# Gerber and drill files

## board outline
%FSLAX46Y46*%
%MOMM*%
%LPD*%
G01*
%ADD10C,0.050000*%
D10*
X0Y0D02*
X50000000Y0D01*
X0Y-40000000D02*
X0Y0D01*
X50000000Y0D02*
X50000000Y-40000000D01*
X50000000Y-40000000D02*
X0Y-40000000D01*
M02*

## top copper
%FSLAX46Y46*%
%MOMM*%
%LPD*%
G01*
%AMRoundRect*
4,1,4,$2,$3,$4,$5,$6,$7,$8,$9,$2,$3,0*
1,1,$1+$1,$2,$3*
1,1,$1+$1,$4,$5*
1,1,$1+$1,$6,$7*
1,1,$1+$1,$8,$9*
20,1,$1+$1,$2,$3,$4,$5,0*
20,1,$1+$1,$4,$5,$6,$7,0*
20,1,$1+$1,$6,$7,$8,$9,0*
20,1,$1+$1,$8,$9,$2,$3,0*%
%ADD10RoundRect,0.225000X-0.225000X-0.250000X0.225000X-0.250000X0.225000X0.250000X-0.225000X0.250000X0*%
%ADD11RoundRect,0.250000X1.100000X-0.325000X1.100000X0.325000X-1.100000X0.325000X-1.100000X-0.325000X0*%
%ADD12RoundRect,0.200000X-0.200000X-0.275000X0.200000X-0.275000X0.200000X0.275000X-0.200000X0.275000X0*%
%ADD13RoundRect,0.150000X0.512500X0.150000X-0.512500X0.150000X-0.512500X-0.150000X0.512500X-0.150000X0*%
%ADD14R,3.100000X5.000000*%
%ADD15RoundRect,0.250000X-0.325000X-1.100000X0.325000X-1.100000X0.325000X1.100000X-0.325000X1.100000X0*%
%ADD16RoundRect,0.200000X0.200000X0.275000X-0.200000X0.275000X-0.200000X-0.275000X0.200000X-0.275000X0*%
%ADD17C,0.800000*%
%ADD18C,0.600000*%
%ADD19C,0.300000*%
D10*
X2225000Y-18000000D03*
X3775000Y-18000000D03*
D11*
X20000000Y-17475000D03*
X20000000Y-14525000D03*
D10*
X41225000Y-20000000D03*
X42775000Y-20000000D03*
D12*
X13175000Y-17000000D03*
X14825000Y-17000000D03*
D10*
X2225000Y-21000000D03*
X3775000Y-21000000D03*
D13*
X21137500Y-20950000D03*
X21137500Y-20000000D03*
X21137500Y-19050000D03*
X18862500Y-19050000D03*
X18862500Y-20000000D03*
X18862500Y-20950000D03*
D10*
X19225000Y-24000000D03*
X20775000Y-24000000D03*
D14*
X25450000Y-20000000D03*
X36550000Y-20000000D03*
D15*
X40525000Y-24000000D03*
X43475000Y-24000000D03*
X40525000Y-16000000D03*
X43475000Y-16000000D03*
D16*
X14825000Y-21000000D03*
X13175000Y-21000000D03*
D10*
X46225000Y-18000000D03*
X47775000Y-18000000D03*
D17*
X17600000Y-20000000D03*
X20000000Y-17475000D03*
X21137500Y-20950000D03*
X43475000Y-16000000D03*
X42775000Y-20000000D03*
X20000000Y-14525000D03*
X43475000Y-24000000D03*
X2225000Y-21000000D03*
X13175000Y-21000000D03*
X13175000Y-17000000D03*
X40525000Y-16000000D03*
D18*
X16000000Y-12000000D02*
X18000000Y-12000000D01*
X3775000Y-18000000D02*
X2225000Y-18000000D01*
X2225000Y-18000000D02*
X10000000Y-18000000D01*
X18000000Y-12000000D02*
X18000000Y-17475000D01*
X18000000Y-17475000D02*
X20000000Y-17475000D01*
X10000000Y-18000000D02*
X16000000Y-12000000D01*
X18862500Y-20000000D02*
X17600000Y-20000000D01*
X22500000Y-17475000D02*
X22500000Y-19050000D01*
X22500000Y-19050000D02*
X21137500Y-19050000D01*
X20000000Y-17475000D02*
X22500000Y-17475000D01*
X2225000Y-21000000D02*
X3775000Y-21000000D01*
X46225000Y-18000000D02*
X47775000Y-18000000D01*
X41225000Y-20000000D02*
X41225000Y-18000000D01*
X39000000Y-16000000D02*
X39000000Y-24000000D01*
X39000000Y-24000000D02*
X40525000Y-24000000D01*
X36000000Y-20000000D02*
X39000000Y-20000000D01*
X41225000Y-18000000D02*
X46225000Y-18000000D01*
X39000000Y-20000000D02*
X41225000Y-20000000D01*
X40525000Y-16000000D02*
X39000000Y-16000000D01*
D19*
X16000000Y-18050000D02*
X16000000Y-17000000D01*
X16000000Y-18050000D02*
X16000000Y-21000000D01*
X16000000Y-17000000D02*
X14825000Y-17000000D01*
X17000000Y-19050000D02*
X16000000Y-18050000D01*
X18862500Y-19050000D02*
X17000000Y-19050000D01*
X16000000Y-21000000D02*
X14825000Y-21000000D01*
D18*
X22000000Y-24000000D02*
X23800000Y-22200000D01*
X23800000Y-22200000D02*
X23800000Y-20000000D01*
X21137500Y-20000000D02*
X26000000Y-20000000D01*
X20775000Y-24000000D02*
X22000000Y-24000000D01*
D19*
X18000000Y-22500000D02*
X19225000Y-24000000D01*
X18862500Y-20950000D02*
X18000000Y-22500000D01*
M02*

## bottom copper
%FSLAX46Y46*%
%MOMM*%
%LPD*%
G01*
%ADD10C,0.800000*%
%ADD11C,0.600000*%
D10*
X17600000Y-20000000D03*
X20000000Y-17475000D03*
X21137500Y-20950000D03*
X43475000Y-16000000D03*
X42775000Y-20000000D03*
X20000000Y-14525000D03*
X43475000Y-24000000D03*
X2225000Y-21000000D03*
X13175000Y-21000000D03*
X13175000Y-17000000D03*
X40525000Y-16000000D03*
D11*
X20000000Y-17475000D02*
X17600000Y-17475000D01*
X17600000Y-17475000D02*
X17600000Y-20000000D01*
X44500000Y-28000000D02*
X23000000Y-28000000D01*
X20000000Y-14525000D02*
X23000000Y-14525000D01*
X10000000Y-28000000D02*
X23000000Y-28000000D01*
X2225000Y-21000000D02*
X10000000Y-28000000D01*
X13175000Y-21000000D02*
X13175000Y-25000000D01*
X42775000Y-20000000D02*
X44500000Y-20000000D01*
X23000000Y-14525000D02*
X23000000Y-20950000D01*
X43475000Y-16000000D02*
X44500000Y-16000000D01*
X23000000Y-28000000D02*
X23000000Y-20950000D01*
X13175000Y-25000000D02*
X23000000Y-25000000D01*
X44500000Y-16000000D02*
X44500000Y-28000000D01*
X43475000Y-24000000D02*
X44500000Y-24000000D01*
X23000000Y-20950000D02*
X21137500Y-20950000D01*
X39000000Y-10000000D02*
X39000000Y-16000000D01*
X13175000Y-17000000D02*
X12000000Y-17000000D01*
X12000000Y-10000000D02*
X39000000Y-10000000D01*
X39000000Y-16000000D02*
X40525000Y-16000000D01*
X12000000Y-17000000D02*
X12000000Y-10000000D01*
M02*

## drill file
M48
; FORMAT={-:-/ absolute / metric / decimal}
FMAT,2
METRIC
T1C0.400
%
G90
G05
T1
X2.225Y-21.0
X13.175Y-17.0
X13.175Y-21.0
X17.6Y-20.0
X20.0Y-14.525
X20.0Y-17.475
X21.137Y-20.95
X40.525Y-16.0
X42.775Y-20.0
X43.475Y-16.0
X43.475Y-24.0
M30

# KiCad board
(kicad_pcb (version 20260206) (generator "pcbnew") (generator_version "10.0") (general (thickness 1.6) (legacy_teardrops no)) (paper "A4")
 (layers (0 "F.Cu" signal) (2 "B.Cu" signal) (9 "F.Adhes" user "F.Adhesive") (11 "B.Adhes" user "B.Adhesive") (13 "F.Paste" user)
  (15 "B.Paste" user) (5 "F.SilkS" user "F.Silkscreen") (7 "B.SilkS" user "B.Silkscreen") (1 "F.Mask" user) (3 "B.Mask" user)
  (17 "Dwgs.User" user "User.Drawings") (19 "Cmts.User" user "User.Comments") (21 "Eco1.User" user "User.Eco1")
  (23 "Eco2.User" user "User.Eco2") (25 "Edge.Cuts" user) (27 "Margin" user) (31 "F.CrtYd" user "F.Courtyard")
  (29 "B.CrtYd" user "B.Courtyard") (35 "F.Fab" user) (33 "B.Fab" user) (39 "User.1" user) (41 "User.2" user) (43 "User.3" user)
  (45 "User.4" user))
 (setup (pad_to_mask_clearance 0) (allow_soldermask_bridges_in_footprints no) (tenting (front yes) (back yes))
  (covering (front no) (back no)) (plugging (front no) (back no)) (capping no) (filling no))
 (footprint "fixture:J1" (layer "F.Cu") (at 3 18)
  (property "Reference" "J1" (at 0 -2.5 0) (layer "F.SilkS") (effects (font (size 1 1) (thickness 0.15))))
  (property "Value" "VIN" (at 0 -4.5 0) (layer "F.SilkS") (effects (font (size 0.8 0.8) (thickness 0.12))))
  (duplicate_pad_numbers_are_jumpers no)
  (pad "1" smd roundrect (at -0.775 0) (size 0.9 0.95) (layers "F.Cu" "F.Mask" "F.Paste") (roundrect_rratio 0.25) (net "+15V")
   (thermal_bridge_angle 45))
  (pad "2" smd roundrect (at 0.775 0) (size 0.9 0.95) (layers "F.Cu" "F.Mask" "F.Paste") (roundrect_rratio 0.25) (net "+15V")
   (thermal_bridge_angle 45)))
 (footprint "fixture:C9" (layer "F.Cu") (at 20 16 90)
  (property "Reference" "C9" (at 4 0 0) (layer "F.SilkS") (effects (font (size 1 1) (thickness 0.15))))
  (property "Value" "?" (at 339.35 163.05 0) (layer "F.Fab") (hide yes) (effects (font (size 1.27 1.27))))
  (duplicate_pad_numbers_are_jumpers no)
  (pad "1" smd roundrect (at -1.475 0 90) (size 1.15 2.7) (layers "F.Cu" "F.Mask" "F.Paste") (roundrect_rratio 0.217391) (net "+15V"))
  (pad "2" smd roundrect (at 1.475 0 90) (size 1.15 2.7) (layers "F.Cu" "F.Mask" "F.Paste") (roundrect_rratio 0.217391) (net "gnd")))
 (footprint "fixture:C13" (layer "F.Cu") (at 42 20)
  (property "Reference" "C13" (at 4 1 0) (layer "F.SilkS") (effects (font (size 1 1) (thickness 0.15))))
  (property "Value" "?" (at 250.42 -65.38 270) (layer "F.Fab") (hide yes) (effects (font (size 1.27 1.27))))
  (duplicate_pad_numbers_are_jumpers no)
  (pad "1" smd roundrect (at -0.775 0) (size 0.9 0.95) (layers "F.Cu" "F.Mask" "F.Paste") (roundrect_rratio 0.25) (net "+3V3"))
  (pad "2" smd roundrect (at 0.775 0) (size 0.9 0.95) (layers "F.Cu" "F.Mask" "F.Paste") (roundrect_rratio 0.25) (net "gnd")))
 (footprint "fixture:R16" (layer "F.Cu") (at 14 17)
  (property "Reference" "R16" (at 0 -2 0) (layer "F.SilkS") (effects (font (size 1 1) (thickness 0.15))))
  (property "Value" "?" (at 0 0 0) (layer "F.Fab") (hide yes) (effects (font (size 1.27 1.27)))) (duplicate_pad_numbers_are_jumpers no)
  (pad "1" smd roundrect (at -0.825 0) (size 0.8 0.95) (layers "F.Cu" "F.Mask" "F.Paste") (roundrect_rratio 0.25) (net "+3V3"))
  (pad "2" smd roundrect (at 0.825 0) (size 0.8 0.95) (layers "F.Cu" "F.Mask" "F.Paste") (roundrect_rratio 0.25) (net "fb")))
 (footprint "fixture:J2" (layer "F.Cu") (at 3 21)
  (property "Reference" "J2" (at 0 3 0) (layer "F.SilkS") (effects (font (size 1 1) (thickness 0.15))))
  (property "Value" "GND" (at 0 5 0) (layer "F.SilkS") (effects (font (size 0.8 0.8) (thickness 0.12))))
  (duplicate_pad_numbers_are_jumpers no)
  (pad "1" smd roundrect (at -0.775 0) (size 0.9 0.95) (layers "F.Cu" "F.Mask" "F.Paste") (roundrect_rratio 0.25) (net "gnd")
   (thermal_bridge_angle 45))
  (pad "2" smd roundrect (at 0.775 0) (size 0.9 0.95) (layers "F.Cu" "F.Mask" "F.Paste") (roundrect_rratio 0.25) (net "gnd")
   (thermal_bridge_angle 45)))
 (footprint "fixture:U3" (layer "F.Cu") (at 20 20 180)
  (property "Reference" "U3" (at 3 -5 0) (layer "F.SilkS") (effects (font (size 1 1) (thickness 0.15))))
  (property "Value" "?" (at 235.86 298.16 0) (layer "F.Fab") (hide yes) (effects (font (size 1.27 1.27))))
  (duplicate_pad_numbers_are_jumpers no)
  (pad "1" smd roundrect (at -1.1375 -0.95 180) (size 1.325 0.6) (layers "F.Cu" "F.Mask" "F.Paste") (roundrect_rratio 0.25) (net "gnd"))
  (pad "2" smd roundrect (at -1.1375 0 180) (size 1.325 0.6) (layers "F.Cu" "F.Mask" "F.Paste") (roundrect_rratio 0.25) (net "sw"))
  (pad "3" smd roundrect (at -1.1375 0.95 180) (size 1.325 0.6) (layers "F.Cu" "F.Mask" "F.Paste") (roundrect_rratio 0.25) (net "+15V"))
  (pad "4" smd roundrect (at 1.1375 0.95 180) (size 1.325 0.6) (layers "F.Cu" "F.Mask" "F.Paste") (roundrect_rratio 0.25) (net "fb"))
  (pad "5" smd roundrect (at 1.1375 0 180) (size 1.325 0.6) (layers "F.Cu" "F.Mask" "F.Paste") (roundrect_rratio 0.25) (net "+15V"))
  (pad "6" smd roundrect (at 1.1375 -0.95 180) (size 1.325 0.6) (layers "F.Cu" "F.Mask" "F.Paste") (roundrect_rratio 0.25) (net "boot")))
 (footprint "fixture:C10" (layer "F.Cu") (at 20 24)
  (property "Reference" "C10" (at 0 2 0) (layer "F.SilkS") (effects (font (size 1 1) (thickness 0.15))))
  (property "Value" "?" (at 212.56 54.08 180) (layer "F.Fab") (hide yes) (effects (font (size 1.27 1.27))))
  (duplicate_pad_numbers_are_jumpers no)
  (pad "1" smd roundrect (at -0.775 0) (size 0.9 0.95) (layers "F.Cu" "F.Mask" "F.Paste") (roundrect_rratio 0.25) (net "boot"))
  (pad "2" smd roundrect (at 0.775 0) (size 0.9 0.95) (layers "F.Cu" "F.Mask" "F.Paste") (roundrect_rratio 0.25) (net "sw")))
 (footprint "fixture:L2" (layer "F.Cu") (at 31 20)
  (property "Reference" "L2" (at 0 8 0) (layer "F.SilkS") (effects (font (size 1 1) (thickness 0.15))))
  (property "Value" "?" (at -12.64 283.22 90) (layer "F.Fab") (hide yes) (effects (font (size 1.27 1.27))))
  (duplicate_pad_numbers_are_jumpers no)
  (pad "1" smd rect (at -5.55 0) (size 3.1 5.0) (layers "F.Cu" "F.Mask" "F.Paste") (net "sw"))
  (pad "2" smd rect (at 5.55 0) (size 3.1 5.0) (layers "F.Cu" "F.Mask" "F.Paste") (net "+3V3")))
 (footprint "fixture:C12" (layer "F.Cu") (at 42 24)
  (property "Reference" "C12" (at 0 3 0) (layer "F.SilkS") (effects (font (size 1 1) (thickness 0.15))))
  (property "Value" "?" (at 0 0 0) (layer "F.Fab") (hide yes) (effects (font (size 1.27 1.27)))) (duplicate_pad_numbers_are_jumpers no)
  (pad "1" smd roundrect (at -1.475 0) (size 1.15 2.7) (layers "F.Cu" "F.Mask" "F.Paste") (roundrect_rratio 0.217391) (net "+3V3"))
  (pad "2" smd roundrect (at 1.475 0) (size 1.15 2.7) (layers "F.Cu" "F.Mask" "F.Paste") (roundrect_rratio 0.217391) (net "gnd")))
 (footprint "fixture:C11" (layer "F.Cu") (at 42 16)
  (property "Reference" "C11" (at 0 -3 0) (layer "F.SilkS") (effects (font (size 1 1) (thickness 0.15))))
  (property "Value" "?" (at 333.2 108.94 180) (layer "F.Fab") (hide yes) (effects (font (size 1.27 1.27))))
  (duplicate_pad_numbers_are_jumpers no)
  (pad "1" smd roundrect (at -1.475 0) (size 1.15 2.7) (layers "F.Cu" "F.Mask" "F.Paste") (roundrect_rratio 0.217391) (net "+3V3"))
  (pad "2" smd roundrect (at 1.475 0) (size 1.15 2.7) (layers "F.Cu" "F.Mask" "F.Paste") (roundrect_rratio 0.217391) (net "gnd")))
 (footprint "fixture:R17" (layer "F.Cu") (at 14 21 180)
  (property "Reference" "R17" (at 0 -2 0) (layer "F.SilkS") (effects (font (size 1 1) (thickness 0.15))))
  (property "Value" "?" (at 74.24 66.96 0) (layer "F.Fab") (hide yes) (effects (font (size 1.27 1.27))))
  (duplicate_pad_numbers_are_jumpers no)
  (pad "1" smd roundrect (at -0.825 0 180) (size 0.8 0.95) (layers "F.Cu" "F.Mask" "F.Paste") (roundrect_rratio 0.25) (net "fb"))
  (pad "2" smd roundrect (at 0.825 0 180) (size 0.8 0.95) (layers "F.Cu" "F.Mask" "F.Paste") (roundrect_rratio 0.25) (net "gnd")))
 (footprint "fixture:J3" (layer "F.Cu") (at 47 18)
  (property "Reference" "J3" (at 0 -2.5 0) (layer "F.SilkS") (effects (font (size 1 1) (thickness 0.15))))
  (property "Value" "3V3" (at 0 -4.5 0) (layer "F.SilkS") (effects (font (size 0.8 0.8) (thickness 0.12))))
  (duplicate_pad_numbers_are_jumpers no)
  (pad "1" smd roundrect (at -0.775 0) (size 0.9 0.95) (layers "F.Cu" "F.Mask" "F.Paste") (roundrect_rratio 0.25) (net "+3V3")
   (thermal_bridge_angle 45))
  (pad "2" smd roundrect (at 0.775 0) (size 0.9 0.95) (layers "F.Cu" "F.Mask" "F.Paste") (roundrect_rratio 0.25) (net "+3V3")
   (thermal_bridge_angle 45)))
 (gr_line (start 0 0) (end 50 0) (stroke (width 0.05) (type default)) (layer "Edge.Cuts"))
 (gr_line (start 0 40) (end 0 0) (stroke (width 0.05) (type default)) (layer "Edge.Cuts"))
 (gr_line (start 50 0) (end 50 40) (stroke (width 0.05) (type default)) (layer "Edge.Cuts"))
 (gr_line (start 50 40) (end 0 40) (stroke (width 0.05) (type default)) (layer "Edge.Cuts"))
 (segment (start 16 12) (end 18 12) (width 0.6) (layer "F.Cu") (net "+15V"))
 (segment (start 3.775 18) (end 2.225 18) (width 0.6) (layer "F.Cu") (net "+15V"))
 (segment (start 2.225 18) (end 10 18) (width 0.6) (layer "F.Cu") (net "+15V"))
 (segment (start 18 12) (end 18 17.475) (width 0.6) (layer "F.Cu") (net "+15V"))
 (segment (start 18 17.475) (end 20 17.475) (width 0.6) (layer "F.Cu") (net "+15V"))
 (segment (start 10 18) (end 16 12) (width 0.6) (layer "F.Cu") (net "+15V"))
 (segment (start 18.8625 20) (end 17.6 20) (width 0.6) (layer "F.Cu") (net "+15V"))
 (segment (start 22.5 17.475) (end 22.5 19.05) (width 0.6) (layer "F.Cu") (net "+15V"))
 (segment (start 22.5 19.05) (end 21.1375 19.05) (width 0.6) (layer "F.Cu") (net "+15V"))
 (segment (start 20 17.475) (end 22.5 17.475) (width 0.6) (layer "F.Cu") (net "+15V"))
 (via (at 17.6 20) (size 0.8) (drill 0.4) (layers "F.Cu" "B.Cu") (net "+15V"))
 (via (at 20 17.475) (size 0.8) (drill 0.4) (layers "F.Cu" "B.Cu") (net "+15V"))
 (segment (start 20 17.475) (end 17.6 17.475) (width 0.6) (layer "B.Cu") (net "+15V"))
 (segment (start 17.6 17.475) (end 17.6 20) (width 0.6) (layer "B.Cu") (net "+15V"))
 (segment (start 2.225 21) (end 3.775 21) (width 0.6) (layer "F.Cu") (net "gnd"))
 (via (at 21.1375 20.95) (size 0.8) (drill 0.4) (layers "F.Cu" "B.Cu") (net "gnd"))
 (via (at 43.475 16) (size 0.8) (drill 0.4) (layers "F.Cu" "B.Cu") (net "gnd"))
 (via (at 42.775 20) (size 0.8) (drill 0.4) (layers "F.Cu" "B.Cu") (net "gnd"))
 (via (at 20 14.525) (size 0.8) (drill 0.4) (layers "F.Cu" "B.Cu") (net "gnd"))
 (via (at 43.475 24) (size 0.8) (drill 0.4) (layers "F.Cu" "B.Cu") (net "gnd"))
 (via (at 2.225 21) (size 0.8) (drill 0.4) (layers "F.Cu" "B.Cu") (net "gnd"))
 (via (at 13.175 21) (size 0.8) (drill 0.4) (layers "F.Cu" "B.Cu") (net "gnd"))
 (segment (start 44.5 28) (end 23 28) (width 0.6) (layer "B.Cu") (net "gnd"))
 (segment (start 20 14.525) (end 23 14.525) (width 0.6) (layer "B.Cu") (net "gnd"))
 (segment (start 10 28) (end 23 28) (width 0.6) (layer "B.Cu") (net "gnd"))
 (segment (start 2.225 21) (end 10 28) (width 0.6) (layer "B.Cu") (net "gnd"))
 (segment (start 13.175 21) (end 13.175 25) (width 0.6) (layer "B.Cu") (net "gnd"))
 (segment (start 42.775 20) (end 44.5 20) (width 0.6) (layer "B.Cu") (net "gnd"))
 (segment (start 23 14.525) (end 23 20.95) (width 0.6) (layer "B.Cu") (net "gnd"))
 (segment (start 43.475 16) (end 44.5 16) (width 0.6) (layer "B.Cu") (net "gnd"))
 (segment (start 23 28) (end 23 20.95) (width 0.6) (layer "B.Cu") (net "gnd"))
 (segment (start 13.175 25) (end 23 25) (width 0.6) (layer "B.Cu") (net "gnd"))
 (segment (start 44.5 16) (end 44.5 28) (width 0.6) (layer "B.Cu") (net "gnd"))
 (segment (start 43.475 24) (end 44.5 24) (width 0.6) (layer "B.Cu") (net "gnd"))
 (segment (start 23 20.95) (end 21.1375 20.95) (width 0.6) (layer "B.Cu") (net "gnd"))
 (segment (start 46.225 18) (end 47.775 18) (width 0.6) (layer "F.Cu") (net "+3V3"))
 (segment (start 41.225 20) (end 41.225 18) (width 0.6) (layer "F.Cu") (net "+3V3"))
 (segment (start 39 16) (end 39 24) (width 0.6) (layer "F.Cu") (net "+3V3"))
 (segment (start 39 24) (end 40.525 24) (width 0.6) (layer "F.Cu") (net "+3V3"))
 (segment (start 36 20) (end 39 20) (width 0.6) (layer "F.Cu") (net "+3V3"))
 (segment (start 41.225 18) (end 46.225 18) (width 0.6) (layer "F.Cu") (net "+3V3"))
 (segment (start 39 20) (end 41.225 20) (width 0.6) (layer "F.Cu") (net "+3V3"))
 (segment (start 40.525 16) (end 39 16) (width 0.6) (layer "F.Cu") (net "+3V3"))
 (via (at 13.175 17) (size 0.8) (drill 0.4) (layers "F.Cu" "B.Cu") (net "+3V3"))
 (via (at 40.525 16) (size 0.8) (drill 0.4) (layers "F.Cu" "B.Cu") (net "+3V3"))
 (segment (start 39 10) (end 39 16) (width 0.6) (layer "B.Cu") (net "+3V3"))
 (segment (start 13.175 17) (end 12 17) (width 0.6) (layer "B.Cu") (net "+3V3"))
 (segment (start 12 10) (end 39 10) (width 0.6) (layer "B.Cu") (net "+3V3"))
 (segment (start 39 16) (end 40.525 16) (width 0.6) (layer "B.Cu") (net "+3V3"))
 (segment (start 12 17) (end 12 10) (width 0.6) (layer "B.Cu") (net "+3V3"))
 (segment (start 16 18.05) (end 16 17) (width 0.3) (layer "F.Cu") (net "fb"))
 (segment (start 16 18.05) (end 16 21) (width 0.3) (layer "F.Cu") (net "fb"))
 (segment (start 16 17) (end 14.825 17) (width 0.3) (layer "F.Cu") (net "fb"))
 (segment (start 17 19.05) (end 16 18.05) (width 0.3) (layer "F.Cu") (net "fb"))
 (segment (start 18.8625 19.05) (end 17 19.05) (width 0.3) (layer "F.Cu") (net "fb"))
 (segment (start 16 21) (end 14.825 21) (width 0.3) (layer "F.Cu") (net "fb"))
 (segment (start 22 24) (end 23.8 22.2) (width 0.6) (layer "F.Cu") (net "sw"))
 (segment (start 23.8 22.2) (end 23.8 20) (width 0.6) (layer "F.Cu") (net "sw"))
 (segment (start 21.1375 20) (end 26 20) (width 0.6) (layer "F.Cu") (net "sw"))
 (segment (start 20.775 24) (end 22 24) (width 0.6) (layer "F.Cu") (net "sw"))
 (segment (start 18 22.5) (end 19.225 24) (width 0.3) (layer "F.Cu") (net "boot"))
 (segment (start 18.8625 20.95) (end 18 22.5) (width 0.3) (layer "F.Cu") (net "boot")))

